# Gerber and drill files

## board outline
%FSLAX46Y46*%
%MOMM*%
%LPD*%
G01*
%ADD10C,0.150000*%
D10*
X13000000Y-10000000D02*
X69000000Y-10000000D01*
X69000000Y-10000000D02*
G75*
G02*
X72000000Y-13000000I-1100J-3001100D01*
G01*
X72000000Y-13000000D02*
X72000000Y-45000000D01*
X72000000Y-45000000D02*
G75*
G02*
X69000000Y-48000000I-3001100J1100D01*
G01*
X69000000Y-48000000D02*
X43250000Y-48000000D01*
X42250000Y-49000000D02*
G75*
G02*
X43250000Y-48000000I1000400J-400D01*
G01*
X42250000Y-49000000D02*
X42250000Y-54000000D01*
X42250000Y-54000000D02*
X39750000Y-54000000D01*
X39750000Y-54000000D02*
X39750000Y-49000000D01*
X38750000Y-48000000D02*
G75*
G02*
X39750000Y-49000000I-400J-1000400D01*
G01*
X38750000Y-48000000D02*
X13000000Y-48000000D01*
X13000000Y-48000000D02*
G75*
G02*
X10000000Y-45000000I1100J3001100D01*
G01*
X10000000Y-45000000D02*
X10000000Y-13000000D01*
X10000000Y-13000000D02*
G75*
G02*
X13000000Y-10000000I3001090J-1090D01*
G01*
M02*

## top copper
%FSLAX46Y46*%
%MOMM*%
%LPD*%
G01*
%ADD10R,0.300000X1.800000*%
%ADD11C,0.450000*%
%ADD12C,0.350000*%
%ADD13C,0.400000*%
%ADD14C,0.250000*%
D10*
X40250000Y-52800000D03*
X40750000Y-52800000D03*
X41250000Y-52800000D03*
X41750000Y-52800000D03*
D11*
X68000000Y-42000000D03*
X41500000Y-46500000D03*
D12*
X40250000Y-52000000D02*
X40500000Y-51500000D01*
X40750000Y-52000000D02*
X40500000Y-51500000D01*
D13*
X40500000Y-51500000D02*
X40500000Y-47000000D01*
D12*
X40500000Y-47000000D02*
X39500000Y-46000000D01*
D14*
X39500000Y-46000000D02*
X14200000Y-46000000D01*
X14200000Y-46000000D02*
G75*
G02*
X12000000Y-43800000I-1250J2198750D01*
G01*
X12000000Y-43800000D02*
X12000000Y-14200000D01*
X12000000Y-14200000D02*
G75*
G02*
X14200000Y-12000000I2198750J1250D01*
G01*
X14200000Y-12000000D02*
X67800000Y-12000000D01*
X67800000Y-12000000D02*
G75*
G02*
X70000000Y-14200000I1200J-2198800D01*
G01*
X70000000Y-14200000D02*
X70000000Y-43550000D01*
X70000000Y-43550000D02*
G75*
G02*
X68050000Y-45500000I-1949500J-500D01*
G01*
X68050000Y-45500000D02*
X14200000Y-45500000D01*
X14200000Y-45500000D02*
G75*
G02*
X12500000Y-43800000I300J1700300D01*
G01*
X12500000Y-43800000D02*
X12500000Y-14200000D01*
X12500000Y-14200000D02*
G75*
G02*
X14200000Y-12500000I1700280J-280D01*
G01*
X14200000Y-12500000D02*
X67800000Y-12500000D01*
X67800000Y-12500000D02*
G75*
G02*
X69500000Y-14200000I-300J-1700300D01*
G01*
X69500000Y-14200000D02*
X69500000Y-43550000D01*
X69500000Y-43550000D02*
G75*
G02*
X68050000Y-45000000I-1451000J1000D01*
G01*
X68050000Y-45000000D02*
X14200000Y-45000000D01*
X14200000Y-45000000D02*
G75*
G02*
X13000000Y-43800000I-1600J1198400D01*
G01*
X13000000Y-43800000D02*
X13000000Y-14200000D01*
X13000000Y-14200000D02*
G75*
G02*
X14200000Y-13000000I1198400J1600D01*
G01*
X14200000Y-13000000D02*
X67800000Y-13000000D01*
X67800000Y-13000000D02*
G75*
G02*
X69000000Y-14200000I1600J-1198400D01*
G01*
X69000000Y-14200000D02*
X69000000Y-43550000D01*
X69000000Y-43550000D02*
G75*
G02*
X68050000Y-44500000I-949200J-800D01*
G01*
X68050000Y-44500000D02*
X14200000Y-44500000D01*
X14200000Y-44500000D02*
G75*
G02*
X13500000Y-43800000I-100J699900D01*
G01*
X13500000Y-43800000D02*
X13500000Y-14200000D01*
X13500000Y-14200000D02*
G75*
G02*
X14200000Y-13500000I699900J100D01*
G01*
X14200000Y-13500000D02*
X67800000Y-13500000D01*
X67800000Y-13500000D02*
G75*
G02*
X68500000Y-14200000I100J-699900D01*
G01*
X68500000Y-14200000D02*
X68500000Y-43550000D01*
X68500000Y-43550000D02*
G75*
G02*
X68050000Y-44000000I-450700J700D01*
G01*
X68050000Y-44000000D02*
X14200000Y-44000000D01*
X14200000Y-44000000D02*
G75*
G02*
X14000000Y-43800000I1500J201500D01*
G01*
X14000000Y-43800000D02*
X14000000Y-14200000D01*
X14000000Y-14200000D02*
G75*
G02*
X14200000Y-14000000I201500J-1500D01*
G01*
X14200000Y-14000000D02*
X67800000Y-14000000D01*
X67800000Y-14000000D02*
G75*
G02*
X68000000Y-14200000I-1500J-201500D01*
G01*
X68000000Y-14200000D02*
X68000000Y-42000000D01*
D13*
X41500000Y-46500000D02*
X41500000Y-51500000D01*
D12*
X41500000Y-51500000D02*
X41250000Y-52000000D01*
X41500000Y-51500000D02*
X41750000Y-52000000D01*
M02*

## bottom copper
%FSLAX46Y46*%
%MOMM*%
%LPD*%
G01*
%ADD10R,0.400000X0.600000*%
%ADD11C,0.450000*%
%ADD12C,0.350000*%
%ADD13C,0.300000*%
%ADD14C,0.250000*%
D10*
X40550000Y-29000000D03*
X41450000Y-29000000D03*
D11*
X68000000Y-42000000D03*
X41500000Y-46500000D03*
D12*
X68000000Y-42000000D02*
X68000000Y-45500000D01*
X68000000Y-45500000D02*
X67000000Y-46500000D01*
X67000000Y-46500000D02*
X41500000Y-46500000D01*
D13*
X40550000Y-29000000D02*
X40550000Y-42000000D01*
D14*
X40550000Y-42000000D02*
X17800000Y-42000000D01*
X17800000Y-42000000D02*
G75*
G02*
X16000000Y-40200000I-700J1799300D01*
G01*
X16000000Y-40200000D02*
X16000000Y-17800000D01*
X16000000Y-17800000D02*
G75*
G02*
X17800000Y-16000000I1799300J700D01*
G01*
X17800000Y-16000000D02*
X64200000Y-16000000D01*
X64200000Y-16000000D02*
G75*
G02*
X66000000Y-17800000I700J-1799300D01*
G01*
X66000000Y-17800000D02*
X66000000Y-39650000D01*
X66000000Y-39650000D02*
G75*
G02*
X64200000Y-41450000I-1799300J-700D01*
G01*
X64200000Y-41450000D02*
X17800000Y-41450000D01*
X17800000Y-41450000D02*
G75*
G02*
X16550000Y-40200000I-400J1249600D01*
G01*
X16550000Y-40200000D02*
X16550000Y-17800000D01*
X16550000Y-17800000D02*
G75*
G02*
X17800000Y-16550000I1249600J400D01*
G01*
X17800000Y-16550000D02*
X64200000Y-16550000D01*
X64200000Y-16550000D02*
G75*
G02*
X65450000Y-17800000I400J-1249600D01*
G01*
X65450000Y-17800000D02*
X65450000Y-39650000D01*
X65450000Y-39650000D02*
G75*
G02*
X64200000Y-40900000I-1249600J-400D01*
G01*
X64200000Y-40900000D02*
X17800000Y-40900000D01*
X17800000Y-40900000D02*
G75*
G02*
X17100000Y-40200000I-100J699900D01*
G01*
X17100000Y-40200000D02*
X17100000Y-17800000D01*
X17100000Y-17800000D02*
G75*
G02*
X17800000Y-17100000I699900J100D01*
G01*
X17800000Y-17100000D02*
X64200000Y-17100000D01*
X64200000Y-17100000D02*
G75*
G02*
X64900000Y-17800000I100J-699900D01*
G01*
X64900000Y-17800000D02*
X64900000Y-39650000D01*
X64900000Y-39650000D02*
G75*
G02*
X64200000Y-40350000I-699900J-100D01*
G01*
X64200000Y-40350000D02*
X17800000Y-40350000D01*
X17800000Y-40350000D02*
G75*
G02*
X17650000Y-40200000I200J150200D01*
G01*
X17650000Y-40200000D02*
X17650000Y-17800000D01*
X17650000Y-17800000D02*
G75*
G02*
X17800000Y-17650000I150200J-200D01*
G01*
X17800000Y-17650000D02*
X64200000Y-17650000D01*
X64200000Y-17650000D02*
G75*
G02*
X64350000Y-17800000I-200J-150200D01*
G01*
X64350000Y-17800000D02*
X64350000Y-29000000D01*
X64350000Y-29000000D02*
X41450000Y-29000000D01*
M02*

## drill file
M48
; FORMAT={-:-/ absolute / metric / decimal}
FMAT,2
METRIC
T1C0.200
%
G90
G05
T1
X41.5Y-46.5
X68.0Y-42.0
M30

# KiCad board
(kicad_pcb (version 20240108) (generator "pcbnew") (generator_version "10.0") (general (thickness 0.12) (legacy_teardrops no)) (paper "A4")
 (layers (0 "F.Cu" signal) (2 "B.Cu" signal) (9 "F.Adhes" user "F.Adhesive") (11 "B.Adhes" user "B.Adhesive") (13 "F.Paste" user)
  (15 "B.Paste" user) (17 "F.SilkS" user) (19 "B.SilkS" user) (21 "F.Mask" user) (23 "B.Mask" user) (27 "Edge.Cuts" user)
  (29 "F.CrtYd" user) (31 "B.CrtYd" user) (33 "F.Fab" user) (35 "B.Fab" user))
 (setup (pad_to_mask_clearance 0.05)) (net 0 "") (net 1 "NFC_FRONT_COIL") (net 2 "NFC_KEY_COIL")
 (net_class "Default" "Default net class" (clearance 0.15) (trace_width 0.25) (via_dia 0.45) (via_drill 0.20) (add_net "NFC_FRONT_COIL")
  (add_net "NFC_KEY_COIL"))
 (gr_line (start 13.000 10.000) (end 69.000 10.000) (stroke (width 0.15) (type solid)) (layer "Edge.Cuts"))
 (gr_arc (start 69.000 10.000) (mid 71.121 10.879) (end 72.000 13.000) (stroke (width 0.15) (type solid)) (layer "Edge.Cuts"))
 (gr_line (start 72.000 13.000) (end 72.000 45.000) (stroke (width 0.15) (type solid)) (layer "Edge.Cuts"))
 (gr_arc (start 72.000 45.000) (mid 71.121 47.121) (end 69.000 48.000) (stroke (width 0.15) (type solid)) (layer "Edge.Cuts"))
 (gr_line (start 69.000 48.000) (end 43.250 48.000) (stroke (width 0.15) (type solid)) (layer "Edge.Cuts"))
 (gr_arc (start 43.250 48.000) (mid 42.543 48.293) (end 42.250 49.000) (stroke (width 0.15) (type solid)) (layer "Edge.Cuts"))
 (gr_line (start 42.250 49.000) (end 42.250 54.000) (stroke (width 0.15) (type solid)) (layer "Edge.Cuts"))
 (gr_line (start 42.250 54.000) (end 39.750 54.000) (stroke (width 0.15) (type solid)) (layer "Edge.Cuts"))
 (gr_line (start 39.750 54.000) (end 39.750 49.000) (stroke (width 0.15) (type solid)) (layer "Edge.Cuts"))
 (gr_arc (start 39.750 49.000) (mid 39.457 48.293) (end 38.750 48.000) (stroke (width 0.15) (type solid)) (layer "Edge.Cuts"))
 (gr_line (start 38.750 48.000) (end 13.000 48.000) (stroke (width 0.15) (type solid)) (layer "Edge.Cuts"))
 (gr_arc (start 13.000 48.000) (mid 10.879 47.121) (end 10.000 45.000) (stroke (width 0.15) (type solid)) (layer "Edge.Cuts"))
 (gr_line (start 10.000 45.000) (end 10.000 13.000) (stroke (width 0.15) (type solid)) (layer "Edge.Cuts"))
 (gr_arc (start 10.000 13.000) (mid 10.879 10.879) (end 13.000 10.000) (stroke (width 0.15) (type solid)) (layer "Edge.Cuts"))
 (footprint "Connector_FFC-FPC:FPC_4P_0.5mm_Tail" (layer "F.Cu") (at 41.0 52.8 0)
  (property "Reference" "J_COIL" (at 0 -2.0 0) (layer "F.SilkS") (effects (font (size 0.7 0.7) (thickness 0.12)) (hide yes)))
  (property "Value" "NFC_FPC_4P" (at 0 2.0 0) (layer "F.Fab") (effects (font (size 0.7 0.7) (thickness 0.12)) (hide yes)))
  (pad "1" smd rect (at -0.750 0.000) (size 0.300 1.800) (layers "F.Cu" "F.Mask") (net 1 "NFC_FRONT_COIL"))
  (pad "2" smd rect (at -0.250 0.000) (size 0.300 1.800) (layers "F.Cu" "F.Mask") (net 1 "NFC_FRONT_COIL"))
  (pad "3" smd rect (at 0.250 0.000) (size 0.300 1.800) (layers "F.Cu" "F.Mask") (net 1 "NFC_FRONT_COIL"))
  (pad "4" smd rect (at 0.750 0.000) (size 0.300 1.800) (layers "F.Cu" "F.Mask") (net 1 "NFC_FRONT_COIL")))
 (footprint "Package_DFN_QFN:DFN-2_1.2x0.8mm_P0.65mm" (layer "B.Cu") (at 41.0 29.0 0)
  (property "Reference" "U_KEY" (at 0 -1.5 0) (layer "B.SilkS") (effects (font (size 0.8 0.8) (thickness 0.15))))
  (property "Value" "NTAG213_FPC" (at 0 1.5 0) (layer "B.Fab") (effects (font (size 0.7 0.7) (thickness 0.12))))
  (pad "1" smd rect (at -0.45 0.0) (size 0.40 0.60) (layers "B.Cu" "B.Mask" "B.Paste") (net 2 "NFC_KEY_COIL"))
  (pad "2" smd rect (at 0.45 0.0) (size 0.40 0.60) (layers "B.Cu" "B.Mask" "B.Paste") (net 2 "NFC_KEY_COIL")))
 (segment (start 40.250 52.000) (end 40.500 51.500) (width 0.350) (layer "F.Cu") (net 1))
 (segment (start 40.750 52.000) (end 40.500 51.500) (width 0.350) (layer "F.Cu") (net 1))
 (segment (start 40.500 51.500) (end 40.500 47.000) (width 0.400) (layer "F.Cu") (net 1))
 (arc (start 40.500 47.000) (mid 40.207 46.707) (end 39.500 46.000) (width 0.350) (layer "F.Cu") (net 1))
 (segment (start 39.500 46.000) (end 14.200 46.000) (width 0.250) (layer "F.Cu") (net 1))
 (arc (start 14.200 46.000) (mid 12.644 45.356) (end 12.000 43.800) (width 0.250) (layer "F.Cu") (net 1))
 (segment (start 12.000 43.800) (end 12.000 14.200) (width 0.250) (layer "F.Cu") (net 1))
 (arc (start 12.000 14.200) (mid 12.644 12.644) (end 14.200 12.000) (width 0.250) (layer "F.Cu") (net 1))
 (segment (start 14.200 12.000) (end 67.800 12.000) (width 0.250) (layer "F.Cu") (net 1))
 (arc (start 67.800 12.000) (mid 69.356 12.644) (end 70.000 14.200) (width 0.250) (layer "F.Cu") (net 1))
 (segment (start 70.000 14.200) (end 70.000 43.550) (width 0.250) (layer "F.Cu") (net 1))
 (arc (start 70.000 43.550) (mid 69.429 44.929) (end 68.050 45.500) (width 0.250) (layer "F.Cu") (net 1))
 (segment (start 68.050 45.500) (end 14.200 45.500) (width 0.250) (layer "F.Cu") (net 1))
 (arc (start 14.200 45.500) (mid 12.998 45.002) (end 12.500 43.800) (width 0.250) (layer "F.Cu") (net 1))
 (segment (start 12.500 43.800) (end 12.500 14.200) (width 0.250) (layer "F.Cu") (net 1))
 (arc (start 12.500 14.200) (mid 12.998 12.998) (end 14.200 12.500) (width 0.250) (layer "F.Cu") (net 1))
 (segment (start 14.200 12.500) (end 67.800 12.500) (width 0.250) (layer "F.Cu") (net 1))
 (arc (start 67.800 12.500) (mid 69.002 12.998) (end 69.500 14.200) (width 0.250) (layer "F.Cu") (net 1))
 (segment (start 69.500 14.200) (end 69.500 43.550) (width 0.250) (layer "F.Cu") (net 1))
 (arc (start 69.500 43.550) (mid 69.075 44.575) (end 68.050 45.000) (width 0.250) (layer "F.Cu") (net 1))
 (segment (start 68.050 45.000) (end 14.200 45.000) (width 0.250) (layer "F.Cu") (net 1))
 (arc (start 14.200 45.000) (mid 13.351 44.649) (end 13.000 43.800) (width 0.250) (layer "F.Cu") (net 1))
 (segment (start 13.000 43.800) (end 13.000 14.200) (width 0.250) (layer "F.Cu") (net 1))
 (arc (start 13.000 14.200) (mid 13.351 13.351) (end 14.200 13.000) (width 0.250) (layer "F.Cu") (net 1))
 (segment (start 14.200 13.000) (end 67.800 13.000) (width 0.250) (layer "F.Cu") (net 1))
 (arc (start 67.800 13.000) (mid 68.649 13.351) (end 69.000 14.200) (width 0.250) (layer "F.Cu") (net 1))
 (segment (start 69.000 14.200) (end 69.000 43.550) (width 0.250) (layer "F.Cu") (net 1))
 (arc (start 69.000 43.550) (mid 68.722 44.222) (end 68.050 44.500) (width 0.250) (layer "F.Cu") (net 1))
 (segment (start 68.050 44.500) (end 14.200 44.500) (width 0.250) (layer "F.Cu") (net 1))
 (arc (start 14.200 44.500) (mid 13.705 44.295) (end 13.500 43.800) (width 0.250) (layer "F.Cu") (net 1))
 (segment (start 13.500 43.800) (end 13.500 14.200) (width 0.250) (layer "F.Cu") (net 1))
 (arc (start 13.500 14.200) (mid 13.705 13.705) (end 14.200 13.500) (width 0.250) (layer "F.Cu") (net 1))
 (segment (start 14.200 13.500) (end 67.800 13.500) (width 0.250) (layer "F.Cu") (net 1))
 (arc (start 67.800 13.500) (mid 68.295 13.705) (end 68.500 14.200) (width 0.250) (layer "F.Cu") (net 1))
 (segment (start 68.500 14.200) (end 68.500 43.550) (width 0.250) (layer "F.Cu") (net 1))
 (arc (start 68.500 43.550) (mid 68.368 43.868) (end 68.050 44.000) (width 0.250) (layer "F.Cu") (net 1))
 (segment (start 68.050 44.000) (end 14.200 44.000) (width 0.250) (layer "F.Cu") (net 1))
 (arc (start 14.200 44.000) (mid 14.059 43.941) (end 14.000 43.800) (width 0.250) (layer "F.Cu") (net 1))
 (segment (start 14.000 43.800) (end 14.000 14.200) (width 0.250) (layer "F.Cu") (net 1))
 (arc (start 14.000 14.200) (mid 14.059 14.059) (end 14.200 14.000) (width 0.250) (layer "F.Cu") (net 1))
 (segment (start 14.200 14.000) (end 67.800 14.000) (width 0.250) (layer "F.Cu") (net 1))
 (arc (start 67.800 14.000) (mid 67.941 14.059) (end 68.000 14.200) (width 0.250) (layer "F.Cu") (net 1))
 (segment (start 68.000 14.200) (end 68.000 42.000) (width 0.250) (layer "F.Cu") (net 1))
 (via (at 68.000 42.000) (size 0.450) (drill 0.200) (layers "F.Cu" "B.Cu") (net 1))
 (via (at 41.500 46.500) (size 0.450) (drill 0.200) (layers "F.Cu" "B.Cu") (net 1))
 (segment (start 68.000 42.000) (end 68.000 45.500) (width 0.350) (layer "B.Cu") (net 1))
 (segment (start 68.000 45.500) (end 67.000 46.500) (width 0.350) (layer "B.Cu") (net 1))
 (segment (start 67.000 46.500) (end 41.500 46.500) (width 0.350) (layer "B.Cu") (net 1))
 (segment (start 41.500 46.500) (end 41.500 51.500) (width 0.400) (layer "F.Cu") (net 1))
 (segment (start 41.500 51.500) (end 41.250 52.000) (width 0.350) (layer "F.Cu") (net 1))
 (segment (start 41.500 51.500) (end 41.750 52.000) (width 0.350) (layer "F.Cu") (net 1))
 (segment (start 40.550 29.000) (end 40.550 42.000) (width 0.300) (layer "B.Cu") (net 2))
 (segment (start 40.550 42.000) (end 17.800 42.000) (width 0.250) (layer "B.Cu") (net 2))
 (arc (start 17.800 42.000) (mid 16.527 41.473) (end 16.000 40.200) (width 0.250) (layer "B.Cu") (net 2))
 (segment (start 16.000 40.200) (end 16.000 17.800) (width 0.250) (layer "B.Cu") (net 2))
 (arc (start 16.000 17.800) (mid 16.527 16.527) (end 17.800 16.000) (width 0.250) (layer "B.Cu") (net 2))
 (segment (start 17.800 16.000) (end 64.200 16.000) (width 0.250) (layer "B.Cu") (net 2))
 (arc (start 64.200 16.000) (mid 65.473 16.527) (end 66.000 17.800) (width 0.250) (layer "B.Cu") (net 2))
 (segment (start 66.000 17.800) (end 66.000 39.650) (width 0.250) (layer "B.Cu") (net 2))
 (arc (start 66.000 39.650) (mid 65.473 40.923) (end 64.200 41.450) (width 0.250) (layer "B.Cu") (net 2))
 (segment (start 64.200 41.450) (end 17.800 41.450) (width 0.250) (layer "B.Cu") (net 2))
 (arc (start 17.800 41.450) (mid 16.916 41.084) (end 16.550 40.200) (width 0.250) (layer "B.Cu") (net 2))
 (segment (start 16.550 40.200) (end 16.550 17.800) (width 0.250) (layer "B.Cu") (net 2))
 (arc (start 16.550 17.800) (mid 16.916 16.916) (end 17.800 16.550) (width 0.250) (layer "B.Cu") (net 2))
 (segment (start 17.800 16.550) (end 64.200 16.550) (width 0.250) (layer "B.Cu") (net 2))
 (arc (start 64.200 16.550) (mid 65.084 16.916) (end 65.450 17.800) (width 0.250) (layer "B.Cu") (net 2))
 (segment (start 65.450 17.800) (end 65.450 39.650) (width 0.250) (layer "B.Cu") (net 2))
 (arc (start 65.450 39.650) (mid 65.084 40.534) (end 64.200 40.900) (width 0.250) (layer "B.Cu") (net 2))
 (segment (start 64.200 40.900) (end 17.800 40.900) (width 0.250) (layer "B.Cu") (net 2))
 (arc (start 17.800 40.900) (mid 17.305 40.695) (end 17.100 40.200) (width 0.250) (layer "B.Cu") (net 2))
 (segment (start 17.100 40.200) (end 17.100 17.800) (width 0.250) (layer "B.Cu") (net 2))
 (arc (start 17.100 17.800) (mid 17.305 17.305) (end 17.800 17.100) (width 0.250) (layer "B.Cu") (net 2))
 (segment (start 17.800 17.100) (end 64.200 17.100) (width 0.250) (layer "B.Cu") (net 2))
 (arc (start 64.200 17.100) (mid 64.695 17.305) (end 64.900 17.800) (width 0.250) (layer "B.Cu") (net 2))
 (segment (start 64.900 17.800) (end 64.900 39.650) (width 0.250) (layer "B.Cu") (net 2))
 (arc (start 64.900 39.650) (mid 64.695 40.145) (end 64.200 40.350) (width 0.250) (layer "B.Cu") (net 2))
 (segment (start 64.200 40.350) (end 17.800 40.350) (width 0.250) (layer "B.Cu") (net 2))
 (arc (start 17.800 40.350) (mid 17.694 40.306) (end 17.650 40.200) (width 0.250) (layer "B.Cu") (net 2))
 (segment (start 17.650 40.200) (end 17.650 17.800) (width 0.250) (layer "B.Cu") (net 2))
 (arc (start 17.650 17.800) (mid 17.694 17.694) (end 17.800 17.650) (width 0.250) (layer "B.Cu") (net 2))
 (segment (start 17.800 17.650) (end 64.200 17.650) (width 0.250) (layer "B.Cu") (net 2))
 (arc (start 64.200 17.650) (mid 64.306 17.694) (end 64.350 17.800) (width 0.250) (layer "B.Cu") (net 2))
 (segment (start 64.350 17.800) (end 64.350 29.000) (width 0.250) (layer "B.Cu") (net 2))
 (segment (start 64.350 29.000) (end 41.450 29.000) (width 0.250) (layer "B.Cu") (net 2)))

